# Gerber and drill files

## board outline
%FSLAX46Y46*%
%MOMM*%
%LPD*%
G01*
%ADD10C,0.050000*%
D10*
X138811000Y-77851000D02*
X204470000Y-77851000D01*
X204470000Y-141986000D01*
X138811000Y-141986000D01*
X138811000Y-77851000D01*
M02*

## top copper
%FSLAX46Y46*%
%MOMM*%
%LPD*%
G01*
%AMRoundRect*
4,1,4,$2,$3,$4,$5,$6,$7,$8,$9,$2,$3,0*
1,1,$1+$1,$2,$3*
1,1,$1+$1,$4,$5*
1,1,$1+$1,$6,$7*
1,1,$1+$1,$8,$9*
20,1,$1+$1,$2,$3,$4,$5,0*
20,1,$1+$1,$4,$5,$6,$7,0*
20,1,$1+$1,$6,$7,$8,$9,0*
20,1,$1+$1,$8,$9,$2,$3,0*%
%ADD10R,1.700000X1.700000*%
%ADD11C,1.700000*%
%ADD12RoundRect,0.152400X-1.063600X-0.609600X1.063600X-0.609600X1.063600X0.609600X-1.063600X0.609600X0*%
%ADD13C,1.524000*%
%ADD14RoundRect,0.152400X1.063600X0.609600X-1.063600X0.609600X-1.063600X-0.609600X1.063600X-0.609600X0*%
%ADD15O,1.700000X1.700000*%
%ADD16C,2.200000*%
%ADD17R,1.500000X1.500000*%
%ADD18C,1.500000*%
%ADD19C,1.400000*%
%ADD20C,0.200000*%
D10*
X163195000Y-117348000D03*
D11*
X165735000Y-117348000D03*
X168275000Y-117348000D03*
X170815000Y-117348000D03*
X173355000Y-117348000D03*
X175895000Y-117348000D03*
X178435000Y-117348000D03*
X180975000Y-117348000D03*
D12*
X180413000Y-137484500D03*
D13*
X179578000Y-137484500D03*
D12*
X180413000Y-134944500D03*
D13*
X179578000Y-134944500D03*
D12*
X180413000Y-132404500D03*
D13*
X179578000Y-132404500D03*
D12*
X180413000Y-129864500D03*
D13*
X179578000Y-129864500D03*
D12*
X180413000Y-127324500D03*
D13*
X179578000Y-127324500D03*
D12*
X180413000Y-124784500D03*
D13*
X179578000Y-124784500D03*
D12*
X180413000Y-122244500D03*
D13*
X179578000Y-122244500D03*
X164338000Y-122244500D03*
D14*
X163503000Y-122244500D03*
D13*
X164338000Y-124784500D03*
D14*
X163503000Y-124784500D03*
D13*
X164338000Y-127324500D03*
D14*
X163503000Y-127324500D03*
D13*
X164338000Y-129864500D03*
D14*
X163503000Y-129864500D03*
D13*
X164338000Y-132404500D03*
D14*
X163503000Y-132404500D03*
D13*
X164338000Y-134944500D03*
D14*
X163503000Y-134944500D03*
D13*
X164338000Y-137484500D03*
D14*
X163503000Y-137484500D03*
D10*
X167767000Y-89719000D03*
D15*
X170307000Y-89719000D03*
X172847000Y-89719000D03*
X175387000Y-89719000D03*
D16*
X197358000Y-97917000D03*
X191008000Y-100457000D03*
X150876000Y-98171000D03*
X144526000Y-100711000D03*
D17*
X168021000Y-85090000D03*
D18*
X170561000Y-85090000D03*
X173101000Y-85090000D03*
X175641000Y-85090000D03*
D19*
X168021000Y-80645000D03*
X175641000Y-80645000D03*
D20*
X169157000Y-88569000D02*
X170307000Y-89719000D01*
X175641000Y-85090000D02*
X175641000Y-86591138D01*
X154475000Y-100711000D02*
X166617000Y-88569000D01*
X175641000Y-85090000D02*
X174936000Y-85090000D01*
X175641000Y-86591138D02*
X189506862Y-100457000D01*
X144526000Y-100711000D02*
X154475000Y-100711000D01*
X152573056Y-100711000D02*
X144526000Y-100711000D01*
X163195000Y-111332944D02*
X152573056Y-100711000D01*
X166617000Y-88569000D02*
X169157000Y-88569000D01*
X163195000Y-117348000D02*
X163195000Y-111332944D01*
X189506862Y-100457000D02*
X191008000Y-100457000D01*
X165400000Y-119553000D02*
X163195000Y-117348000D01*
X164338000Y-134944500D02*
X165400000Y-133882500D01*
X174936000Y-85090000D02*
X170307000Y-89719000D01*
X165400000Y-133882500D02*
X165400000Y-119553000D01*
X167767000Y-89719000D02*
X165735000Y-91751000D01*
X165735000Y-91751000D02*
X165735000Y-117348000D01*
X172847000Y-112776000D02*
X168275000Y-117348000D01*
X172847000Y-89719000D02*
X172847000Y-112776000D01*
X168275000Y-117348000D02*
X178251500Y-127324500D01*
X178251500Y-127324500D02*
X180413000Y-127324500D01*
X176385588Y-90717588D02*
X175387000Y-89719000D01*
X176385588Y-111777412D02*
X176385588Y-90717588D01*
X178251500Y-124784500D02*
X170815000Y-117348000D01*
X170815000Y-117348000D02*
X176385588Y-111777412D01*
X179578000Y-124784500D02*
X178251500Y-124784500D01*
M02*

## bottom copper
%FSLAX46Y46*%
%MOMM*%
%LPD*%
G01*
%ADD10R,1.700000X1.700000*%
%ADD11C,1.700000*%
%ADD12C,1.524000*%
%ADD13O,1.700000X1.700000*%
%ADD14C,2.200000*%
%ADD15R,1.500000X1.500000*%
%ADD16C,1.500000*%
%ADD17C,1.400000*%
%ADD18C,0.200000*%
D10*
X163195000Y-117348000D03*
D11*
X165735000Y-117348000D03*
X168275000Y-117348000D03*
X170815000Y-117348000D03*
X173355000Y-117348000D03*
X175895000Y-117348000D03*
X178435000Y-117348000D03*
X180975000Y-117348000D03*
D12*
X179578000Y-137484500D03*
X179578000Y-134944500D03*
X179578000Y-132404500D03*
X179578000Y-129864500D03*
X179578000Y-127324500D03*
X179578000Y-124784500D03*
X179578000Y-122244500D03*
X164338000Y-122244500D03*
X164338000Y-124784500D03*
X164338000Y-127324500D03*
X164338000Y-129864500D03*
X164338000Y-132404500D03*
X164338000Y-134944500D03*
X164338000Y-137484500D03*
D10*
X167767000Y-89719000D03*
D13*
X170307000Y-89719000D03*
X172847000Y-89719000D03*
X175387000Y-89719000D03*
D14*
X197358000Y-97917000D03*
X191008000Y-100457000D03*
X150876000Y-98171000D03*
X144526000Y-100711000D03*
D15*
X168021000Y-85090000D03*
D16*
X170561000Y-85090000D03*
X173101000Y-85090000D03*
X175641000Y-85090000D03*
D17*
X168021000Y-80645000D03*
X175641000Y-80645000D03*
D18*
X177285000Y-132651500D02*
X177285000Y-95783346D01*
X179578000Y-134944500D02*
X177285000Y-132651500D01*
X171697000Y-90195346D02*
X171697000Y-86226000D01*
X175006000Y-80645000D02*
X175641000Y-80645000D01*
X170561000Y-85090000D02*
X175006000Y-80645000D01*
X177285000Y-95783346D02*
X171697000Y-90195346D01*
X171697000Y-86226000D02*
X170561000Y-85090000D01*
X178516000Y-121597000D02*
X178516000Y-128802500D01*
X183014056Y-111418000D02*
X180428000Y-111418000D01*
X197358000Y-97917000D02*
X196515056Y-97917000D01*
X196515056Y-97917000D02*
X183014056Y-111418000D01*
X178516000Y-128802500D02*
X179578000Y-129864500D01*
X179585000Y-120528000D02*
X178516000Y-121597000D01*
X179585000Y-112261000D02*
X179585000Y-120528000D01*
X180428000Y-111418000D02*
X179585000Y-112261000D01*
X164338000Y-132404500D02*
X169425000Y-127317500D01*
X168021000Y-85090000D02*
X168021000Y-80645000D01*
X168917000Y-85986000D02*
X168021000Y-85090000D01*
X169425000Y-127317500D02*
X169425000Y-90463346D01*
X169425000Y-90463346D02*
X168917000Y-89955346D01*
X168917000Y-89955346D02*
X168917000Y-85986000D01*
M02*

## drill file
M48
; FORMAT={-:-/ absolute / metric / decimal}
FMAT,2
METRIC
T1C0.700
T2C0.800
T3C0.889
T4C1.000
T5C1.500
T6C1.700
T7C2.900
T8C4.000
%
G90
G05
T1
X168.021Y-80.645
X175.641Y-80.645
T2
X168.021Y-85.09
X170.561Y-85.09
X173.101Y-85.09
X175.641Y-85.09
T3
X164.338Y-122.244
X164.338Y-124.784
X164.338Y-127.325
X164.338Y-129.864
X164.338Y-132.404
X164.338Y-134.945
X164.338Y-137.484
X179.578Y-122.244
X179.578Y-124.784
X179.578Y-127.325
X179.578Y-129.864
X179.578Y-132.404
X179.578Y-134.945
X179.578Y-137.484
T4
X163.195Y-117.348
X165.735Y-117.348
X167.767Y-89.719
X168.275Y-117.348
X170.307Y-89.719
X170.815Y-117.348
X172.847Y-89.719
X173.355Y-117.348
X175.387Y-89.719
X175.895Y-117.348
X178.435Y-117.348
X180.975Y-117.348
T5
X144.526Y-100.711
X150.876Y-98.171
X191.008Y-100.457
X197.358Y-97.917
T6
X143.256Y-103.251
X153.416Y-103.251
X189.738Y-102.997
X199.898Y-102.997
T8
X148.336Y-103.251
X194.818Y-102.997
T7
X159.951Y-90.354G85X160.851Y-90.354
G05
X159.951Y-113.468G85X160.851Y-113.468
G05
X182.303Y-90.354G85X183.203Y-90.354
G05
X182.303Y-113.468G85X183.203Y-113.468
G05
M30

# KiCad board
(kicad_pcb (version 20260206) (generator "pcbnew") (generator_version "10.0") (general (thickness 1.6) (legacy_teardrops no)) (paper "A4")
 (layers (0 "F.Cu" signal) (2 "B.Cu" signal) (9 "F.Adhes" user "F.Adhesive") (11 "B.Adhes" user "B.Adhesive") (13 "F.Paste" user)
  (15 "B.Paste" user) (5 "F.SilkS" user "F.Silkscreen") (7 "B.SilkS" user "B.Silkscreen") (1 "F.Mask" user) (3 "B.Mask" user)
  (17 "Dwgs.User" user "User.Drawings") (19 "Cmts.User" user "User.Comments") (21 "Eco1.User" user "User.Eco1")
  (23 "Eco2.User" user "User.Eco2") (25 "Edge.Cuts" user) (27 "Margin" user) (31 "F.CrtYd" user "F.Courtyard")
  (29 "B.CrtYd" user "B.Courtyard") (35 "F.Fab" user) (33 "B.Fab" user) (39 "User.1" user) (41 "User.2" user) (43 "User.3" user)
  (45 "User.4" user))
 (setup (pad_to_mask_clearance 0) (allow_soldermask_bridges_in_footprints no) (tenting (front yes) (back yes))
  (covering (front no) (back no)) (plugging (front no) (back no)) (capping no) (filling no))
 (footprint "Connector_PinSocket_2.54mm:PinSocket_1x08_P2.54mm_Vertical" (layer "F.Cu") (at 163.195 117.348 90)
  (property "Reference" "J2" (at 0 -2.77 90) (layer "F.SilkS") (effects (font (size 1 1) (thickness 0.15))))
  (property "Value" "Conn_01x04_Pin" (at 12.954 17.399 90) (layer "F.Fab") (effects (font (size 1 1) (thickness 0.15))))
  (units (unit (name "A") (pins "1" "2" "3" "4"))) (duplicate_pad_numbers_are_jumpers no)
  (pad "1" thru_hole rect (at 0 0 90) (size 1.7 1.7) (drill 1) (layers "*.Cu" "*.Mask") (remove_unused_layers no) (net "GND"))
  (pad "2" thru_hole circle (at 0 2.54 90) (size 1.7 1.7) (drill 1) (layers "*.Cu" "*.Mask") (remove_unused_layers no) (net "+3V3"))
  (pad "3" thru_hole circle (at 0 5.08 90) (size 1.7 1.7) (drill 1) (layers "*.Cu" "*.Mask") (remove_unused_layers no) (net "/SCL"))
  (pad "4" thru_hole circle (at 0 7.62 90) (size 1.7 1.7) (drill 1) (layers "*.Cu" "*.Mask") (remove_unused_layers no) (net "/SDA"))
  (pad "5" thru_hole circle (at 0 10.16 90) (size 1.7 1.7) (drill 1) (layers "*.Cu" "*.Mask") (remove_unused_layers no))
  (pad "6" thru_hole circle (at 0 12.7 90) (size 1.7 1.7) (drill 1) (layers "*.Cu" "*.Mask") (remove_unused_layers no))
  (pad "7" thru_hole circle (at 0 15.24 90) (size 1.7 1.7) (drill 1) (layers "*.Cu" "*.Mask") (remove_unused_layers no))
  (pad "8" thru_hole circle (at 0 17.78 90) (size 1.7 1.7) (drill 1) (layers "*.Cu" "*.Mask") (remove_unused_layers no)))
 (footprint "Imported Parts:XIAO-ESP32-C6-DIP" (layer "F.Cu") (at 171.958 129.8645 -90)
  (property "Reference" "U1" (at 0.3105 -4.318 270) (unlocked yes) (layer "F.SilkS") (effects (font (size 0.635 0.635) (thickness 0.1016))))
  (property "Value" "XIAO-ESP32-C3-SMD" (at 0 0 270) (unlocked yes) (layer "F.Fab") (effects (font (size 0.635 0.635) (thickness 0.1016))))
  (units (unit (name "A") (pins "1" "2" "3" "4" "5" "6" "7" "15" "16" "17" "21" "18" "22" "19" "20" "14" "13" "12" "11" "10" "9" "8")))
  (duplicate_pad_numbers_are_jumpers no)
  (pad "1" smd roundrect (at 7.62 -8.455) (size 2.432 1.524) (layers "F.Cu" "F.Mask") (roundrect_rratio 0.1)
   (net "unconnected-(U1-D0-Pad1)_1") (thermal_bridge_angle 45))
  (pad "1" thru_hole circle (at 7.62 -7.62) (size 1.524 1.524) (drill 0.889) (layers "*.Cu" "*.Mask") (remove_unused_layers no)
   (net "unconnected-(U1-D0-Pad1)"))
  (pad "2" smd roundrect (at 5.08 -8.455) (size 2.432 1.524) (layers "F.Cu" "F.Mask") (roundrect_rratio 0.1) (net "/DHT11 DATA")
   (thermal_bridge_angle 45))
  (pad "2" thru_hole circle (at 5.08 -7.62) (size 1.524 1.524) (drill 0.889) (layers "*.Cu" "*.Mask") (remove_unused_layers no)
   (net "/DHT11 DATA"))
  (pad "3" smd roundrect (at 2.54 -8.455) (size 2.432 1.524) (layers "F.Cu" "F.Mask") (roundrect_rratio 0.1) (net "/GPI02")
   (thermal_bridge_angle 45))
  (pad "3" thru_hole circle (at 2.54 -7.62) (size 1.524 1.524) (drill 0.889) (layers "*.Cu" "*.Mask") (remove_unused_layers no)
   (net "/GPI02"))
  (pad "4" smd roundrect (at 0 -8.455) (size 2.432 1.524) (layers "F.Cu" "F.Mask") (roundrect_rratio 0.1) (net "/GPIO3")
   (thermal_bridge_angle 45))
  (pad "4" thru_hole circle (at 0 -7.62) (size 1.524 1.524) (drill 0.889) (layers "*.Cu" "*.Mask") (remove_unused_layers no) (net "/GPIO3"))
  (pad "5" smd roundrect (at -2.54 -8.455) (size 2.432 1.524) (layers "F.Cu" "F.Mask") (roundrect_rratio 0.1) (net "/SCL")
   (thermal_bridge_angle 45))
  (pad "5" thru_hole circle (at -2.54 -7.62) (size 1.524 1.524) (drill 0.889) (layers "*.Cu" "*.Mask") (remove_unused_layers no)
   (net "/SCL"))
  (pad "6" smd roundrect (at -5.08 -8.455) (size 2.432 1.524) (layers "F.Cu" "F.Mask") (roundrect_rratio 0.1) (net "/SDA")
   (thermal_bridge_angle 45))
  (pad "6" thru_hole circle (at -5.08 -7.62) (size 1.524 1.524) (drill 0.889) (layers "*.Cu" "*.Mask") (remove_unused_layers no)
   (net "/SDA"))
  (pad "7" smd roundrect (at -7.62 -8.455) (size 2.432 1.524) (layers "F.Cu" "F.Mask") (roundrect_rratio 0.1)
   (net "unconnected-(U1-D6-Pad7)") (thermal_bridge_angle 45))
  (pad "7" thru_hole circle (at -7.62 -7.62) (size 1.524 1.524) (drill 0.889) (layers "*.Cu" "*.Mask") (remove_unused_layers no)
   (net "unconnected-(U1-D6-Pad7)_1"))
  (pad "8" thru_hole circle (at -7.62 7.62 180) (size 1.524 1.524) (drill 0.889) (layers "*.Cu" "*.Mask") (remove_unused_layers no)
   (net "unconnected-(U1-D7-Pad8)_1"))
  (pad "8" smd roundrect (at -7.62 8.455 180) (size 2.432 1.524) (layers "F.Cu" "F.Mask") (roundrect_rratio 0.1)
   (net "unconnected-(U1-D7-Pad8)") (thermal_bridge_angle 45))
  (pad "9" thru_hole circle (at -5.08 7.62 180) (size 1.524 1.524) (drill 0.889) (layers "*.Cu" "*.Mask") (remove_unused_layers no)
   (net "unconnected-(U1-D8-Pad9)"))
  (pad "9" smd roundrect (at -5.08 8.455 180) (size 2.432 1.524) (layers "F.Cu" "F.Mask") (roundrect_rratio 0.1)
   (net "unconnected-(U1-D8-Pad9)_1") (thermal_bridge_angle 45))
  (pad "10" thru_hole circle (at -2.54 7.62 180) (size 1.524 1.524) (drill 0.889) (layers "*.Cu" "*.Mask") (remove_unused_layers no)
   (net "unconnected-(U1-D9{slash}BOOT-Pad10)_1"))
  (pad "10" smd roundrect (at -2.54 8.455 180) (size 2.432 1.524) (layers "F.Cu" "F.Mask") (roundrect_rratio 0.1)
   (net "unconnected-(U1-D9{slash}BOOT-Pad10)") (thermal_bridge_angle 45))
  (pad "11" thru_hole circle (at 0 7.62 180) (size 1.524 1.524) (drill 0.889) (layers "*.Cu" "*.Mask") (remove_unused_layers no)
   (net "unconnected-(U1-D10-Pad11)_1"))
  (pad "11" smd roundrect (at 0 8.455 180) (size 2.432 1.524) (layers "F.Cu" "F.Mask") (roundrect_rratio 0.1)
   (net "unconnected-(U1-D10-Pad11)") (thermal_bridge_angle 45))
  (pad "12" thru_hole circle (at 2.54 7.62 180) (size 1.524 1.524) (drill 0.889) (layers "*.Cu" "*.Mask") (remove_unused_layers no)
   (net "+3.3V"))
  (pad "12" smd roundrect (at 2.54 8.455 180) (size 2.432 1.524) (layers "F.Cu" "F.Mask") (roundrect_rratio 0.1) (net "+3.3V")
   (thermal_bridge_angle 45))
  (pad "13" thru_hole circle (at 5.08 7.62 180) (size 1.524 1.524) (drill 0.889) (layers "*.Cu" "*.Mask") (remove_unused_layers no)
   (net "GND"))
  (pad "13" smd roundrect (at 5.08 8.455 180) (size 2.432 1.524) (layers "F.Cu" "F.Mask") (roundrect_rratio 0.1) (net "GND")
   (thermal_bridge_angle 45))
  (pad "14" thru_hole circle (at 7.62 7.62 180) (size 1.524 1.524) (drill 0.889) (layers "*.Cu" "*.Mask") (remove_unused_layers no)
   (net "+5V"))
  (pad "14" smd roundrect (at 7.62 8.455 180) (size 2.432 1.524) (layers "F.Cu" "F.Mask") (roundrect_rratio 0.1) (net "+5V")
   (thermal_bridge_angle 45)))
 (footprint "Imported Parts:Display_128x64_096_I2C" (layer "F.Cu") (at 171.577 89.719)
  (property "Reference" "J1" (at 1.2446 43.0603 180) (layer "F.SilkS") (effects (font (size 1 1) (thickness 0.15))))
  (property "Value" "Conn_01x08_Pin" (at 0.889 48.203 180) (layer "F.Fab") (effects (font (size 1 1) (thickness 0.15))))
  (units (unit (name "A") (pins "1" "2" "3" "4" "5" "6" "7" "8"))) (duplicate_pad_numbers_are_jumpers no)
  (pad "" np_thru_hole oval (at -11.176 0.635) (size 3.8 2.9) (drill oval 3.8 2.9) (layers "*.Cu" "*.Mask"))
  (pad "" np_thru_hole oval (at -11.176 23.749) (size 3.8 2.9) (drill oval 3.8 2.9) (layers "*.Cu" "*.Mask"))
  (pad "" np_thru_hole oval (at 11.176 0.635) (size 3.8 2.9) (drill oval 3.8 2.9) (layers "*.Cu" "*.Mask"))
  (pad "" np_thru_hole oval (at 11.176 23.749) (size 3.8 2.9) (drill oval 3.8 2.9) (layers "*.Cu" "*.Mask"))
  (pad "1" thru_hole rect (at -3.81 0 90) (size 1.7 1.7) (drill 1) (layers "*.Cu" "*.Mask") (remove_unused_layers no) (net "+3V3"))
  (pad "2" thru_hole oval (at -1.27 0 90) (size 1.7 1.7) (drill 1) (layers "*.Cu" "*.Mask") (remove_unused_layers no) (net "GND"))
  (pad "3" thru_hole oval (at 1.27 0 90) (size 1.7 1.7) (drill 1) (layers "*.Cu" "*.Mask") (remove_unused_layers no) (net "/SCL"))
  (pad "4" thru_hole oval (at 3.81 0 90) (size 1.7 1.7) (drill 1) (layers "*.Cu" "*.Mask") (remove_unused_layers no) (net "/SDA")))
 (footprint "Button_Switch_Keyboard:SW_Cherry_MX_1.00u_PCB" (layer "F.Cu") (at 197.358 97.917)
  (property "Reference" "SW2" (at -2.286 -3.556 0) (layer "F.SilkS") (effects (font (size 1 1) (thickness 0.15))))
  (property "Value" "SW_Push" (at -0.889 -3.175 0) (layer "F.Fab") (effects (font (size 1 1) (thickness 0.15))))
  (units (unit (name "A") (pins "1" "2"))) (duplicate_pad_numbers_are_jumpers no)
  (pad "" np_thru_hole circle (at -7.62 5.08) (size 1.7 1.7) (drill 1.7) (layers "*.Cu" "*.Mask"))
  (pad "" np_thru_hole circle (at -2.54 5.08) (size 4 4) (drill 4) (layers "*.Cu" "*.Mask"))
  (pad "" np_thru_hole circle (at 2.54 5.08) (size 1.7 1.7) (drill 1.7) (layers "*.Cu" "*.Mask"))
  (pad "1" thru_hole circle (at 0 0) (size 2.2 2.2) (drill 1.5) (layers "*.Cu" "*.Mask") (remove_unused_layers no) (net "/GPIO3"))
  (pad "2" thru_hole circle (at -6.35 2.54) (size 2.2 2.2) (drill 1.5) (layers "*.Cu" "*.Mask") (remove_unused_layers no) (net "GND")))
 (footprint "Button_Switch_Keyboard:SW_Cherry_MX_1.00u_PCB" (layer "F.Cu") (at 150.876 98.171)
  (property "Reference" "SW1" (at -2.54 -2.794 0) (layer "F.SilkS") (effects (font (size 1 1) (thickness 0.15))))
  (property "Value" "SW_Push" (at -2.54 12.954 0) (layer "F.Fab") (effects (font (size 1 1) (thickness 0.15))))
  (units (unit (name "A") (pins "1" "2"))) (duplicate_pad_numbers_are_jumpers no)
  (pad "" np_thru_hole circle (at -7.62 5.08) (size 1.7 1.7) (drill 1.7) (layers "*.Cu" "*.Mask"))
  (pad "" np_thru_hole circle (at -2.54 5.08) (size 4 4) (drill 4) (layers "*.Cu" "*.Mask"))
  (pad "" np_thru_hole circle (at 2.54 5.08) (size 1.7 1.7) (drill 1.7) (layers "*.Cu" "*.Mask"))
  (pad "1" thru_hole circle (at 0 0) (size 2.2 2.2) (drill 1.5) (layers "*.Cu" "*.Mask") (remove_unused_layers no) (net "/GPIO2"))
  (pad "2" thru_hole circle (at -6.35 2.54) (size 2.2 2.2) (drill 1.5) (layers "*.Cu" "*.Mask") (remove_unused_layers no) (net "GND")))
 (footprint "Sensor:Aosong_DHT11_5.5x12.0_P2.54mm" (layer "F.Cu") (at 168.021 85.09 90)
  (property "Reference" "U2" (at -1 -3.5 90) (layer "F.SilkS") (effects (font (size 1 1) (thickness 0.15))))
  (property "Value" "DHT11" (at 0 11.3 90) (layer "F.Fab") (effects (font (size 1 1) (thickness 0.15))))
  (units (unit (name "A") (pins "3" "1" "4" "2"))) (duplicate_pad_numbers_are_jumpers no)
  (pad "1" thru_hole rect (at 0 0 90) (size 1.5 1.5) (drill 0.8) (layers "*.Cu" "*.Mask") (remove_unused_layers no) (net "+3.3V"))
  (pad "2" thru_hole circle (at 0 2.54 90) (size 1.5 1.5) (drill 0.8) (layers "*.Cu" "*.Mask") (remove_unused_layers no) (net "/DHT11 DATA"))
  (pad "3" thru_hole circle (at 0 5.08 90) (size 1.5 1.5) (drill 0.8) (layers "*.Cu" "*.Mask") (remove_unused_layers no)
   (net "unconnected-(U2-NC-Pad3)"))
  (pad "4" thru_hole circle (at 0 7.62 90) (size 1.5 1.5) (drill 0.8) (layers "*.Cu" "*.Mask") (remove_unused_layers no) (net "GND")))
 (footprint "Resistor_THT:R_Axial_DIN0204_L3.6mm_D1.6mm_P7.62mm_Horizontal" (layer "F.Cu") (at 168.021 80.645)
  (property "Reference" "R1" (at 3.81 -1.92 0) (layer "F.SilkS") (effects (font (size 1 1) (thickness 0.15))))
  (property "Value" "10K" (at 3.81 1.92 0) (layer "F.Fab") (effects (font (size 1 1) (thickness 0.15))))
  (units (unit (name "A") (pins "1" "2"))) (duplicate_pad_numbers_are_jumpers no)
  (pad "1" thru_hole circle (at 0 0) (size 1.4 1.4) (drill 0.7) (layers "*.Cu" "*.Mask") (remove_unused_layers no) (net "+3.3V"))
  (pad "2" thru_hole circle (at 7.62 0) (size 1.4 1.4) (drill 0.7) (layers "*.Cu" "*.Mask") (remove_unused_layers no) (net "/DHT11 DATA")))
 (gr_rect (start 138.811 77.851) (end 204.47 141.986) (stroke (width 0.05) (type default)) (fill no) (layer "Edge.Cuts"))
 (segment (start 169.157 88.569) (end 170.307 89.719) (width 0.2) (layer "F.Cu") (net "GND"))
 (segment (start 175.641 85.09) (end 175.641 86.591138) (width 0.2) (layer "F.Cu") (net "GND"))
 (segment (start 154.475 100.711) (end 166.617 88.569) (width 0.2) (layer "F.Cu") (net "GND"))
 (segment (start 175.641 85.09) (end 174.936 85.09) (width 0.2) (layer "F.Cu") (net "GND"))
 (segment (start 175.641 86.591138) (end 189.506862 100.457) (width 0.2) (layer "F.Cu") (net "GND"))
 (segment (start 144.526 100.711) (end 154.475 100.711) (width 0.2) (layer "F.Cu") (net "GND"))
 (segment (start 152.573056 100.711) (end 144.526 100.711) (width 0.2) (layer "F.Cu") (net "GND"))
 (segment (start 163.195 111.332944) (end 152.573056 100.711) (width 0.2) (layer "F.Cu") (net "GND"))
 (segment (start 166.617 88.569) (end 169.157 88.569) (width 0.2) (layer "F.Cu") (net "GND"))
 (segment (start 163.195 117.348) (end 163.195 111.332944) (width 0.2) (layer "F.Cu") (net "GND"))
 (segment (start 189.506862 100.457) (end 191.008 100.457) (width 0.2) (layer "F.Cu") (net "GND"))
 (segment (start 165.4 119.553) (end 163.195 117.348) (width 0.2) (layer "F.Cu") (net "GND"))
 (segment (start 164.338 134.9445) (end 165.4 133.8825) (width 0.2) (layer "F.Cu") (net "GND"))
 (segment (start 174.936 85.09) (end 170.307 89.719) (width 0.2) (layer "F.Cu") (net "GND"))
 (segment (start 165.4 133.8825) (end 165.4 119.553) (width 0.2) (layer "F.Cu") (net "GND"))
 (segment (start 167.767 89.719) (end 165.735 91.751) (width 0.2) (layer "F.Cu") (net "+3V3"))
 (segment (start 165.735 91.751) (end 165.735 117.348) (width 0.2) (layer "F.Cu") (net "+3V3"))
 (segment (start 172.847 112.776) (end 168.275 117.348) (width 0.2) (layer "F.Cu") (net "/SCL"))
 (segment (start 172.847 89.719) (end 172.847 112.776) (width 0.2) (layer "F.Cu") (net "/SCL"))
 (segment (start 168.275 117.348) (end 178.2515 127.3245) (width 0.2) (layer "F.Cu") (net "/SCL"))
 (segment (start 178.2515 127.3245) (end 180.413 127.3245) (width 0.2) (layer "F.Cu") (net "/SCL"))
 (segment (start 176.385588 90.717588) (end 175.387 89.719) (width 0.2) (layer "F.Cu") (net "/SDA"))
 (segment (start 176.385588 111.777412) (end 176.385588 90.717588) (width 0.2) (layer "F.Cu") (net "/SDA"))
 (segment (start 178.2515 124.7845) (end 170.815 117.348) (width 0.2) (layer "F.Cu") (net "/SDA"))
 (segment (start 170.815 117.348) (end 176.385588 111.777412) (width 0.2) (layer "F.Cu") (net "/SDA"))
 (segment (start 179.578 124.7845) (end 178.2515 124.7845) (width 0.2) (layer "F.Cu") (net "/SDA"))
 (segment (start 177.285 132.6515) (end 177.285 95.783346) (width 0.2) (layer "B.Cu") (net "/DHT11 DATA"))
 (segment (start 179.578 134.9445) (end 177.285 132.6515) (width 0.2) (layer "B.Cu") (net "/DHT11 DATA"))
 (segment (start 171.697 90.195346) (end 171.697 86.226) (width 0.2) (layer "B.Cu") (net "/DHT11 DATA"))
 (segment (start 175.006 80.645) (end 175.641 80.645) (width 0.2) (layer "B.Cu") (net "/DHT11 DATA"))
 (segment (start 170.561 85.09) (end 175.006 80.645) (width 0.2) (layer "B.Cu") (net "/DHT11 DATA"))
 (segment (start 177.285 95.783346) (end 171.697 90.195346) (width 0.2) (layer "B.Cu") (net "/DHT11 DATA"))
 (segment (start 171.697 86.226) (end 170.561 85.09) (width 0.2) (layer "B.Cu") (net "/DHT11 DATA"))
 (segment (start 178.516 121.597) (end 178.516 128.8025) (width 0.2) (layer "B.Cu") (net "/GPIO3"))
 (segment (start 183.014056 111.418) (end 180.428 111.418) (width 0.2) (layer "B.Cu") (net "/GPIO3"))
 (segment (start 197.358 97.917) (end 196.515056 97.917) (width 0.2) (layer "B.Cu") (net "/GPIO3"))
 (segment (start 196.515056 97.917) (end 183.014056 111.418) (width 0.2) (layer "B.Cu") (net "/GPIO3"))
 (segment (start 178.516 128.8025) (end 179.578 129.8645) (width 0.2) (layer "B.Cu") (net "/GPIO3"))
 (segment (start 179.585 120.528) (end 178.516 121.597) (width 0.2) (layer "B.Cu") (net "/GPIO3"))
 (segment (start 179.585 112.261) (end 179.585 120.528) (width 0.2) (layer "B.Cu") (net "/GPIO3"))
 (segment (start 180.428 111.418) (end 179.585 112.261) (width 0.2) (layer "B.Cu") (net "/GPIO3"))
 (segment (start 164.338 132.4045) (end 169.425 127.3175) (width 0.2) (layer "B.Cu") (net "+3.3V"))
 (segment (start 168.021 85.09) (end 168.021 80.645) (width 0.2) (layer "B.Cu") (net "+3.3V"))
 (segment (start 168.917 85.986) (end 168.021 85.09) (width 0.2) (layer "B.Cu") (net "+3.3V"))
 (segment (start 169.425 127.3175) (end 169.425 90.463346) (width 0.2) (layer "B.Cu") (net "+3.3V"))
 (segment (start 169.425 90.463346) (end 168.917 89.955346) (width 0.2) (layer "B.Cu") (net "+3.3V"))
 (segment (start 168.917 89.955346) (end 168.917 85.986) (width 0.2) (layer "B.Cu") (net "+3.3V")))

